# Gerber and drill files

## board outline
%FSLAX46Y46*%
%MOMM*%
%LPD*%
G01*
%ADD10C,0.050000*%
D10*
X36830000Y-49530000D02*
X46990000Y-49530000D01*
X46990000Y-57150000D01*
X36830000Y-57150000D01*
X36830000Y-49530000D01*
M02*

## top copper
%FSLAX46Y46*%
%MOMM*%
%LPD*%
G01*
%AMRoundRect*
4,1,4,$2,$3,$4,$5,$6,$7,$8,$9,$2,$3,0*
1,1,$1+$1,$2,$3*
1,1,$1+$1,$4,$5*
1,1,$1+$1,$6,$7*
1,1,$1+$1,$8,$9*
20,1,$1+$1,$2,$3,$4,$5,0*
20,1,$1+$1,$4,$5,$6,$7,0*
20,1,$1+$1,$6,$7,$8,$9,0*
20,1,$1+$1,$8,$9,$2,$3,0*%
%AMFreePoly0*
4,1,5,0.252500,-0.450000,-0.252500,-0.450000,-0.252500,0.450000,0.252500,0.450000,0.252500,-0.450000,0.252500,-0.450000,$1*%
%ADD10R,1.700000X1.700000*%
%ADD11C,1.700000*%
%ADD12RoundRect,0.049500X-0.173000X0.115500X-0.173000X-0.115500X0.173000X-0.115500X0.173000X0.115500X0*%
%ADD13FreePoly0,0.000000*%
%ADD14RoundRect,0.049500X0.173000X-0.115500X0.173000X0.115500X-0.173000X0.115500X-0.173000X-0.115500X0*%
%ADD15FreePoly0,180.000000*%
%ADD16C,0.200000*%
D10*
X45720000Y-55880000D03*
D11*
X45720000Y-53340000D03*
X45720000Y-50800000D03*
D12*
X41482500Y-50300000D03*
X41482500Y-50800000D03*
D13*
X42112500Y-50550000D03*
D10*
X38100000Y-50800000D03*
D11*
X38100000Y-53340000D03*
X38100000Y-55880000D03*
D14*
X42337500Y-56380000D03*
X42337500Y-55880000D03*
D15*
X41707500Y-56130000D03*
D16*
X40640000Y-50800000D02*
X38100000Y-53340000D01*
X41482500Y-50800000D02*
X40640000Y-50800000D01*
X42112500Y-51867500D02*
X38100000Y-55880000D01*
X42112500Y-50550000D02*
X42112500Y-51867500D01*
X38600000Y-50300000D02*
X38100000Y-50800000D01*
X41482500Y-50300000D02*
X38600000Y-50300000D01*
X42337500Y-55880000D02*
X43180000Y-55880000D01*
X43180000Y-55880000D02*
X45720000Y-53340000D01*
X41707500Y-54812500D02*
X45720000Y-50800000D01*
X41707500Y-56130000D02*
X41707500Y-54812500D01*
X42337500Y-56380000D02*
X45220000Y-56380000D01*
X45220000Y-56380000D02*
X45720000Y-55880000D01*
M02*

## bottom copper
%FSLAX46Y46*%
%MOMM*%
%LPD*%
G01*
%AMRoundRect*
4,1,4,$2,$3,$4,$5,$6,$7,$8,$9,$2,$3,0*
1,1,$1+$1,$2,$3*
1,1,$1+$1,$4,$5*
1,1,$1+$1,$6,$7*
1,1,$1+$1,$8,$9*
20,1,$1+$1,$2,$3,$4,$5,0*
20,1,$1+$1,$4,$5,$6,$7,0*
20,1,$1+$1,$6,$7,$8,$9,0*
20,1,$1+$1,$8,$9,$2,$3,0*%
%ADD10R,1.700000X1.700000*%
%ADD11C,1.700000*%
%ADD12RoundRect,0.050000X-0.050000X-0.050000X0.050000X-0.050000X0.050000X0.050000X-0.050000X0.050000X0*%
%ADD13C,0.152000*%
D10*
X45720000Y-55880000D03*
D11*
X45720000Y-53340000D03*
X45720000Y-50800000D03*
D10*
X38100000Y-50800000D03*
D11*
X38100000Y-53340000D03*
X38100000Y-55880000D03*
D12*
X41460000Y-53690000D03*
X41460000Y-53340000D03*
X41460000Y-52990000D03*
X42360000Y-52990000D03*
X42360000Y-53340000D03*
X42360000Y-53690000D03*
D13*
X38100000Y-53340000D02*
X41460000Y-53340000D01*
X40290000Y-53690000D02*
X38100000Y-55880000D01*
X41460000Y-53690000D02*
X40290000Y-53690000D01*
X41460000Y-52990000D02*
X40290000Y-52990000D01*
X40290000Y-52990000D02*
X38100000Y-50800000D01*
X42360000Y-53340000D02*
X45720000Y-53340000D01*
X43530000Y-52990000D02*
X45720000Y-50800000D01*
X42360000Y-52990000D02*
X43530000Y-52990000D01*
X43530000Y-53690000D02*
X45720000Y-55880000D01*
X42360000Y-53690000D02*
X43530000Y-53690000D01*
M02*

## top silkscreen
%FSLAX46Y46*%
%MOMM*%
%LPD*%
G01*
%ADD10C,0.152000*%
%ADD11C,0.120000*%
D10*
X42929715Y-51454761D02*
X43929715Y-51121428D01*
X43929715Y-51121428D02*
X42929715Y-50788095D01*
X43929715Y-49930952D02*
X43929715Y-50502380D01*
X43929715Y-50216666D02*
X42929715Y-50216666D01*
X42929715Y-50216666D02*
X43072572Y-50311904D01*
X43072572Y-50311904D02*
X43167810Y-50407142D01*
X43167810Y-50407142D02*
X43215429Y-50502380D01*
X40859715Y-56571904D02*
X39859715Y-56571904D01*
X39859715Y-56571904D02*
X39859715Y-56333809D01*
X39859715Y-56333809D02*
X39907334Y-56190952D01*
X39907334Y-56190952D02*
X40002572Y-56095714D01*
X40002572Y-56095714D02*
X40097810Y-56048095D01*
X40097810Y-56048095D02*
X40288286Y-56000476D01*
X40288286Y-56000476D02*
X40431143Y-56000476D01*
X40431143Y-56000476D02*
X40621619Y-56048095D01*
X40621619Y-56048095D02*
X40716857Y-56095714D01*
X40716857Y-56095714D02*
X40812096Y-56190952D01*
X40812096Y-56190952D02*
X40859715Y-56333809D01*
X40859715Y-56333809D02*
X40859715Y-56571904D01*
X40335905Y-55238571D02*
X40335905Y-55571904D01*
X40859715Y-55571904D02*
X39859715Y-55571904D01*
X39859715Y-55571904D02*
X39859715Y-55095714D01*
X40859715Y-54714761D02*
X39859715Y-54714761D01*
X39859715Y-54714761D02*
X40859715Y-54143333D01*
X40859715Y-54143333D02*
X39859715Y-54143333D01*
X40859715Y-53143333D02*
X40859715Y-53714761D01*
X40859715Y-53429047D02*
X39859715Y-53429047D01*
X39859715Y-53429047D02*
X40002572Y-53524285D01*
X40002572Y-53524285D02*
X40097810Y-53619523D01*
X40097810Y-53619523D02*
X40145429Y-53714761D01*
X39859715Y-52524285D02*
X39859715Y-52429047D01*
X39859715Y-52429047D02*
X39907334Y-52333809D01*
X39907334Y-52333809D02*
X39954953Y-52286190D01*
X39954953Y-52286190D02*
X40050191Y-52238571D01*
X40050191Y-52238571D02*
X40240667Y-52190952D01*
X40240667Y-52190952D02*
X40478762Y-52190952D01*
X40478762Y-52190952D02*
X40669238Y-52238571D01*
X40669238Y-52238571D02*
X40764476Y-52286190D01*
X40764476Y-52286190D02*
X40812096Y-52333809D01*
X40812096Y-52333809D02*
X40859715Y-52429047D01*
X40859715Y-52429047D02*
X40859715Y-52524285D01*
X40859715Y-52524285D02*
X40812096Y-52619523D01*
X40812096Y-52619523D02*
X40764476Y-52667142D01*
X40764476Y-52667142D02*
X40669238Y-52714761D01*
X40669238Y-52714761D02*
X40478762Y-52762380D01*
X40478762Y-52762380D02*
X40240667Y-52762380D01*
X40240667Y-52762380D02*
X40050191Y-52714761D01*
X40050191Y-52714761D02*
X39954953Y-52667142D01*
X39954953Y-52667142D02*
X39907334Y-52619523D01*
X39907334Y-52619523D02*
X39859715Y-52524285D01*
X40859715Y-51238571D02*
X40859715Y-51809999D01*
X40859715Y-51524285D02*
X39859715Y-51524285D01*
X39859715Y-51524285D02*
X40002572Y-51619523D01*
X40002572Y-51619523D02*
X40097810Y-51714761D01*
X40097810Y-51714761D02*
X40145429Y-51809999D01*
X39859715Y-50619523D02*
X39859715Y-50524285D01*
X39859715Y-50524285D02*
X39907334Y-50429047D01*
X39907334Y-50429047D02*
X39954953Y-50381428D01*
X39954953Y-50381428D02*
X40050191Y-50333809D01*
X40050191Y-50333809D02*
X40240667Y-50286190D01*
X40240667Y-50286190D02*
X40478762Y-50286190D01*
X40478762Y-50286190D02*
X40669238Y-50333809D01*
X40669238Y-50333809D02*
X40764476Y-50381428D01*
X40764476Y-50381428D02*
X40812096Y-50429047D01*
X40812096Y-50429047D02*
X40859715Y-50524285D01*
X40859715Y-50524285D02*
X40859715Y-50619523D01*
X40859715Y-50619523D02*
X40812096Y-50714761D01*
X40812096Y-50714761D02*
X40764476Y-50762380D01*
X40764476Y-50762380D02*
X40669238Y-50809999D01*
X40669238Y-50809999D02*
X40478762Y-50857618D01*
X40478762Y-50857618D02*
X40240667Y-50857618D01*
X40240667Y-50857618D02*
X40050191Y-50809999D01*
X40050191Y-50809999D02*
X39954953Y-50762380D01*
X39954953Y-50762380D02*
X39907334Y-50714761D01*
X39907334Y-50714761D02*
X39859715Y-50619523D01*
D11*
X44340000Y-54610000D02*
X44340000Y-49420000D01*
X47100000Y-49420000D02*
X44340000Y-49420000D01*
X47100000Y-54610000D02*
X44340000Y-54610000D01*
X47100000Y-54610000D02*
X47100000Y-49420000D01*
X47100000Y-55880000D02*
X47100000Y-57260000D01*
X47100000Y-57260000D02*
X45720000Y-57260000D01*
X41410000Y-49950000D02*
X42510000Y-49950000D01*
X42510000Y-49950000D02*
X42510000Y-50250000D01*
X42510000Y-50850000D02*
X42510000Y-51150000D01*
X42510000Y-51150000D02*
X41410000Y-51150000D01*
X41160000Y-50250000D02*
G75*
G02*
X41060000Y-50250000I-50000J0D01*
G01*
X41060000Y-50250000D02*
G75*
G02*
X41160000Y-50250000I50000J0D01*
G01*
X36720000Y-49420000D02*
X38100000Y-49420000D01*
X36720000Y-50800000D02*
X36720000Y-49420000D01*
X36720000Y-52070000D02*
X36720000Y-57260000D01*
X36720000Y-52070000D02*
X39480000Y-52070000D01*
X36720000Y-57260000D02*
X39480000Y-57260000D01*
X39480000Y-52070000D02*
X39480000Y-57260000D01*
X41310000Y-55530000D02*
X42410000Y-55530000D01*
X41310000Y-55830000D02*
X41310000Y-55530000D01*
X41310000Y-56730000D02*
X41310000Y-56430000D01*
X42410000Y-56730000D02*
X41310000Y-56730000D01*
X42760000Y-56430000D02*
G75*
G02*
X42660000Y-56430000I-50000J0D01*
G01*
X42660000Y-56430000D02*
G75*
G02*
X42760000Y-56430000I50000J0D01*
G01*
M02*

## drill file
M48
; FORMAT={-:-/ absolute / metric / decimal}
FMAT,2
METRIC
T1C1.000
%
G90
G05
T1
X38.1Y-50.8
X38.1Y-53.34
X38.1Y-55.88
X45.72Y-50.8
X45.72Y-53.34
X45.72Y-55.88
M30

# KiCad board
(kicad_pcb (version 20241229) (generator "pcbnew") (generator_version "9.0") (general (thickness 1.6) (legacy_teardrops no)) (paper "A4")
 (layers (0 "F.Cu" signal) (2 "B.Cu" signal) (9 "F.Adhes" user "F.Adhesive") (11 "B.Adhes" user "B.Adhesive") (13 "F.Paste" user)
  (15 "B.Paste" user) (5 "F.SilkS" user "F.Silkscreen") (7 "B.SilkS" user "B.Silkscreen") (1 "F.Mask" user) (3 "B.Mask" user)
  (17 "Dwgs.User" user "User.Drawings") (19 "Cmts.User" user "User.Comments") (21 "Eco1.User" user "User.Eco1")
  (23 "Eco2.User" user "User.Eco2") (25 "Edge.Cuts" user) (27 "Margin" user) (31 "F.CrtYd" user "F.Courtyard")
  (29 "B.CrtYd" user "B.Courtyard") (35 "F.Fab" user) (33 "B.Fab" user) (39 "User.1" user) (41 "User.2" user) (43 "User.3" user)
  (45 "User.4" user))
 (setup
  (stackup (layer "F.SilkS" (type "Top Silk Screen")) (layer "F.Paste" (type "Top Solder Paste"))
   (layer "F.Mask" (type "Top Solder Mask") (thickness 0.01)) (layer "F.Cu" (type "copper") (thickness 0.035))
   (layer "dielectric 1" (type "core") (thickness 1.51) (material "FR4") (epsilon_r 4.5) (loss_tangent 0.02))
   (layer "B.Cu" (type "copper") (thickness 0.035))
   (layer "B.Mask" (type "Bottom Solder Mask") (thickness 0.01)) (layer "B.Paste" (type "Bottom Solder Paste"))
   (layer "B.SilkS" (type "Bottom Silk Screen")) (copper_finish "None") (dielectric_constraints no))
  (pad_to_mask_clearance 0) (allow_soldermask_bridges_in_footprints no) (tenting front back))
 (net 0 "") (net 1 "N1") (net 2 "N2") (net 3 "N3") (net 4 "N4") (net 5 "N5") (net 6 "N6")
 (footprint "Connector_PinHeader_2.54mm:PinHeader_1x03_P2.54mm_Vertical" (layer "F.Cu") (at 45.72 55.88 180)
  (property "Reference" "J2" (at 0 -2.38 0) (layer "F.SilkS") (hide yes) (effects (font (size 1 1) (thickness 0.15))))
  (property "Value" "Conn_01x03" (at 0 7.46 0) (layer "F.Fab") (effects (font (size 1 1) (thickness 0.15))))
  (fp_line (start 1.38 1.27) (end 1.38 6.46) (stroke (width 0.12) (type solid)) (layer "F.SilkS"))
  (fp_line (start -1.38 6.46) (end 1.38 6.46) (stroke (width 0.12) (type solid)) (layer "F.SilkS"))
  (fp_line (start -1.38 1.27) (end 1.38 1.27) (stroke (width 0.12) (type solid)) (layer "F.SilkS"))
  (fp_line (start -1.38 1.27) (end -1.38 6.46) (stroke (width 0.12) (type solid)) (layer "F.SilkS"))
  (fp_line (start -1.38 0) (end -1.38 -1.38) (stroke (width 0.12) (type solid)) (layer "F.SilkS"))
  (fp_line (start -1.38 -1.38) (end 0 -1.38) (stroke (width 0.12) (type solid)) (layer "F.SilkS"))
  (pad "1" thru_hole rect (at 0 0 180) (size 1.7 1.7) (drill 1) (layers "*.Cu" "*.Mask") (remove_unused_layers no) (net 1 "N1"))
  (pad "2" thru_hole circle (at 0 2.54 180) (size 1.7 1.7) (drill 1) (layers "*.Cu" "*.Mask") (remove_unused_layers no) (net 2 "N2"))
  (pad "3" thru_hole circle (at 0 5.08 180) (size 1.7 1.7) (drill 1) (layers "*.Cu" "*.Mask") (remove_unused_layers no) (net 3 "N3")))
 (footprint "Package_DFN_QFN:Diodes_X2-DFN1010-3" (layer "F.Cu") (at 41.91 50.55)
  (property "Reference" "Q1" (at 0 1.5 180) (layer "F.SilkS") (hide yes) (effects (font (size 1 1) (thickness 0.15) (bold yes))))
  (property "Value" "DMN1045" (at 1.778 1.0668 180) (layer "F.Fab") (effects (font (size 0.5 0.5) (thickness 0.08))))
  (fp_line (start -0.5 -0.6) (end 0.6 -0.6) (stroke (width 0.12) (type default)) (layer "F.SilkS"))
  (fp_line (start 0.6 -0.6) (end 0.6 -0.3) (stroke (width 0.12) (type default)) (layer "F.SilkS"))
  (fp_line (start 0.6 0.3) (end 0.6 0.6) (stroke (width 0.12) (type default)) (layer "F.SilkS"))
  (fp_line (start 0.6 0.6) (end -0.5 0.6) (stroke (width 0.12) (type default)) (layer "F.SilkS"))
  (fp_circle (center -0.8 -0.3) (end -0.75 -0.3) (stroke (width 0.12) (type solid)) (fill no) (layer "F.SilkS"))
  (pad "1" smd roundrect (at -0.4275 -0.25 270) (size 0.33 0.445) (layers "F.Cu" "F.Mask" "F.Paste") (roundrect_rratio 0.15) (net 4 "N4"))
  (pad "2" smd roundrect (at -0.4275 0.25 270) (size 0.33 0.445) (layers "F.Cu" "F.Mask" "F.Paste") (roundrect_rratio 0.15) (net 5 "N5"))
  (pad "3" smd custom (at 0.2025 0) (size 0.505 0.9) (layers "F.Cu" "F.Mask" "F.Paste") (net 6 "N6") (solder_paste_margin -0.06)
   (zone_connect 0) (thermal_bridge_angle 45) (options (clearance outline) (anchor rect)) (primitives)))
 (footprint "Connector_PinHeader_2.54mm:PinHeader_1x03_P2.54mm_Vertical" (layer "F.Cu") (at 38.1 50.8)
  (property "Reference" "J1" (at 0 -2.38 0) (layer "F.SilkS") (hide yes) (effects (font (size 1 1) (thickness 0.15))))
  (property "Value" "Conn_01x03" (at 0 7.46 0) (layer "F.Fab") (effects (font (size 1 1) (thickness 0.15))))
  (fp_line (start -1.38 -1.38) (end 0 -1.38) (stroke (width 0.12) (type solid)) (layer "F.SilkS"))
  (fp_line (start -1.38 0) (end -1.38 -1.38) (stroke (width 0.12) (type solid)) (layer "F.SilkS"))
  (fp_line (start -1.38 1.27) (end -1.38 6.46) (stroke (width 0.12) (type solid)) (layer "F.SilkS"))
  (fp_line (start -1.38 1.27) (end 1.38 1.27) (stroke (width 0.12) (type solid)) (layer "F.SilkS"))
  (fp_line (start -1.38 6.46) (end 1.38 6.46) (stroke (width 0.12) (type solid)) (layer "F.SilkS"))
  (fp_line (start 1.38 1.27) (end 1.38 6.46) (stroke (width 0.12) (type solid)) (layer "F.SilkS"))
  (pad "1" thru_hole rect (at 0 0) (size 1.7 1.7) (drill 1) (layers "*.Cu" "*.Mask") (remove_unused_layers no) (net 4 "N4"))
  (pad "2" thru_hole circle (at 0 2.54) (size 1.7 1.7) (drill 1) (layers "*.Cu" "*.Mask") (remove_unused_layers no) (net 5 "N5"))
  (pad "3" thru_hole circle (at 0 5.08) (size 1.7 1.7) (drill 1) (layers "*.Cu" "*.Mask") (remove_unused_layers no) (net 6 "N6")))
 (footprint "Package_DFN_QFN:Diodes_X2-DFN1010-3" (layer "F.Cu") (at 41.91 56.13 180)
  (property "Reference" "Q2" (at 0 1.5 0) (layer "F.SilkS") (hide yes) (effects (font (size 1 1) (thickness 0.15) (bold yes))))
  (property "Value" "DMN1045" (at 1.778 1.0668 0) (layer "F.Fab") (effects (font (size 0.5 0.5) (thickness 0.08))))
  (fp_line (start 0.6 0.6) (end -0.5 0.6) (stroke (width 0.12) (type default)) (layer "F.SilkS"))
  (fp_line (start 0.6 0.3) (end 0.6 0.6) (stroke (width 0.12) (type default)) (layer "F.SilkS"))
  (fp_line (start 0.6 -0.6) (end 0.6 -0.3) (stroke (width 0.12) (type default)) (layer "F.SilkS"))
  (fp_line (start -0.5 -0.6) (end 0.6 -0.6) (stroke (width 0.12) (type default)) (layer "F.SilkS"))
  (fp_circle (center -0.8 -0.3) (end -0.75 -0.3) (stroke (width 0.12) (type solid)) (fill no) (layer "F.SilkS"))
  (pad "1" smd roundrect (at -0.4275 -0.25 90) (size 0.33 0.445) (layers "F.Cu" "F.Mask" "F.Paste") (roundrect_rratio 0.15) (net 1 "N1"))
  (pad "2" smd roundrect (at -0.4275 0.25 90) (size 0.33 0.445) (layers "F.Cu" "F.Mask" "F.Paste") (roundrect_rratio 0.15) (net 2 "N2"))
  (pad "3" smd custom (at 0.2025 0 180) (size 0.505 0.9) (layers "F.Cu" "F.Mask" "F.Paste") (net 3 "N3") (solder_paste_margin -0.06)
   (zone_connect 0) (thermal_bridge_angle 45) (options (clearance outline) (anchor rect)) (primitives)))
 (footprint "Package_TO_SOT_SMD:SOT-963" (layer "B.Cu") (at 41.91 53.34)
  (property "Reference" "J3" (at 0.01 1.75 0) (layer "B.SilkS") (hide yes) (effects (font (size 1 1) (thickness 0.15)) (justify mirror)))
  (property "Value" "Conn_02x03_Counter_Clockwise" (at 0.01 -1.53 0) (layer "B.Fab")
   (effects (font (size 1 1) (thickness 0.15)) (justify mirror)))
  (pad "1" smd roundrect (at -0.45 0.35) (size 0.2 0.2) (layers "B.Cu" "B.Mask" "B.Paste") (roundrect_rratio 0.25) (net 6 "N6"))
  (pad "2" smd roundrect (at -0.45 0) (size 0.2 0.2) (layers "B.Cu" "B.Mask" "B.Paste") (roundrect_rratio 0.25) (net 5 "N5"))
  (pad "3" smd roundrect (at -0.45 -0.35) (size 0.2 0.2) (layers "B.Cu" "B.Mask" "B.Paste") (roundrect_rratio 0.25) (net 4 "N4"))
  (pad "4" smd roundrect (at 0.45 -0.35) (size 0.2 0.2) (layers "B.Cu" "B.Mask" "B.Paste") (roundrect_rratio 0.25) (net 3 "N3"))
  (pad "5" smd roundrect (at 0.45 0) (size 0.2 0.2) (layers "B.Cu" "B.Mask" "B.Paste") (roundrect_rratio 0.25) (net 2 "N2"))
  (pad "6" smd roundrect (at 0.45 0.35) (size 0.2 0.2) (layers "B.Cu" "B.Mask" "B.Paste") (roundrect_rratio 0.25) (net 1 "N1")))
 (gr_rect (start 36.83 49.53) (end 46.99 57.15) (stroke (width 0.05) (type default)) (fill no) (layer "Edge.Cuts"))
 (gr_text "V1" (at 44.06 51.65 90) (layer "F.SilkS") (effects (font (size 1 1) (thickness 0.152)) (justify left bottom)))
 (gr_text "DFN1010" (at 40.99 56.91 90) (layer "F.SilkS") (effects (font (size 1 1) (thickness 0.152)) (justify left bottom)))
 (segment (start 40.64 50.8) (end 38.1 53.34) (width 0.2) (layer "F.Cu") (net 5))
 (segment (start 41.4825 50.8) (end 40.64 50.8) (width 0.2) (layer "F.Cu") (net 5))
 (segment (start 38.1 53.34) (end 41.46 53.34) (width 0.152) (layer "B.Cu") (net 5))
 (segment (start 42.1125 51.8675) (end 38.1 55.88) (width 0.2) (layer "F.Cu") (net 6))
 (segment (start 42.1125 50.55) (end 42.1125 51.8675) (width 0.2) (layer "F.Cu") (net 6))
 (segment (start 40.29 53.69) (end 38.1 55.88) (width 0.152) (layer "B.Cu") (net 6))
 (segment (start 41.46 53.69) (end 40.29 53.69) (width 0.152) (layer "B.Cu") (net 6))
 (segment (start 38.6 50.3) (end 38.1 50.8) (width 0.2) (layer "F.Cu") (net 4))
 (segment (start 41.4825 50.3) (end 38.6 50.3) (width 0.2) (layer "F.Cu") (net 4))
 (segment (start 41.46 52.99) (end 40.29 52.99) (width 0.152) (layer "B.Cu") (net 4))
 (segment (start 40.29 52.99) (end 38.1 50.8) (width 0.152) (layer "B.Cu") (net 4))
 (segment (start 42.3375 55.88) (end 43.18 55.88) (width 0.2) (layer "F.Cu") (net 2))
 (segment (start 43.18 55.88) (end 45.72 53.34) (width 0.2) (layer "F.Cu") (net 2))
 (segment (start 42.36 53.34) (end 45.72 53.34) (width 0.152) (layer "B.Cu") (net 2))
 (segment (start 41.7075 54.8125) (end 45.72 50.8) (width 0.2) (layer "F.Cu") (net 3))
 (segment (start 41.7075 56.13) (end 41.7075 54.8125) (width 0.2) (layer "F.Cu") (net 3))
 (segment (start 43.53 52.99) (end 45.72 50.8) (width 0.152) (layer "B.Cu") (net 3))
 (segment (start 42.36 52.99) (end 43.53 52.99) (width 0.152) (layer "B.Cu") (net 3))
 (segment (start 42.3375 56.38) (end 45.22 56.38) (width 0.2) (layer "F.Cu") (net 1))
 (segment (start 45.22 56.38) (end 45.72 55.88) (width 0.2) (layer "F.Cu") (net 1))
 (segment (start 43.53 53.69) (end 45.72 55.88) (width 0.152) (layer "B.Cu") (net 1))
 (segment (start 42.36 53.69) (end 43.53 53.69) (width 0.152) (layer "B.Cu") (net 1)))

